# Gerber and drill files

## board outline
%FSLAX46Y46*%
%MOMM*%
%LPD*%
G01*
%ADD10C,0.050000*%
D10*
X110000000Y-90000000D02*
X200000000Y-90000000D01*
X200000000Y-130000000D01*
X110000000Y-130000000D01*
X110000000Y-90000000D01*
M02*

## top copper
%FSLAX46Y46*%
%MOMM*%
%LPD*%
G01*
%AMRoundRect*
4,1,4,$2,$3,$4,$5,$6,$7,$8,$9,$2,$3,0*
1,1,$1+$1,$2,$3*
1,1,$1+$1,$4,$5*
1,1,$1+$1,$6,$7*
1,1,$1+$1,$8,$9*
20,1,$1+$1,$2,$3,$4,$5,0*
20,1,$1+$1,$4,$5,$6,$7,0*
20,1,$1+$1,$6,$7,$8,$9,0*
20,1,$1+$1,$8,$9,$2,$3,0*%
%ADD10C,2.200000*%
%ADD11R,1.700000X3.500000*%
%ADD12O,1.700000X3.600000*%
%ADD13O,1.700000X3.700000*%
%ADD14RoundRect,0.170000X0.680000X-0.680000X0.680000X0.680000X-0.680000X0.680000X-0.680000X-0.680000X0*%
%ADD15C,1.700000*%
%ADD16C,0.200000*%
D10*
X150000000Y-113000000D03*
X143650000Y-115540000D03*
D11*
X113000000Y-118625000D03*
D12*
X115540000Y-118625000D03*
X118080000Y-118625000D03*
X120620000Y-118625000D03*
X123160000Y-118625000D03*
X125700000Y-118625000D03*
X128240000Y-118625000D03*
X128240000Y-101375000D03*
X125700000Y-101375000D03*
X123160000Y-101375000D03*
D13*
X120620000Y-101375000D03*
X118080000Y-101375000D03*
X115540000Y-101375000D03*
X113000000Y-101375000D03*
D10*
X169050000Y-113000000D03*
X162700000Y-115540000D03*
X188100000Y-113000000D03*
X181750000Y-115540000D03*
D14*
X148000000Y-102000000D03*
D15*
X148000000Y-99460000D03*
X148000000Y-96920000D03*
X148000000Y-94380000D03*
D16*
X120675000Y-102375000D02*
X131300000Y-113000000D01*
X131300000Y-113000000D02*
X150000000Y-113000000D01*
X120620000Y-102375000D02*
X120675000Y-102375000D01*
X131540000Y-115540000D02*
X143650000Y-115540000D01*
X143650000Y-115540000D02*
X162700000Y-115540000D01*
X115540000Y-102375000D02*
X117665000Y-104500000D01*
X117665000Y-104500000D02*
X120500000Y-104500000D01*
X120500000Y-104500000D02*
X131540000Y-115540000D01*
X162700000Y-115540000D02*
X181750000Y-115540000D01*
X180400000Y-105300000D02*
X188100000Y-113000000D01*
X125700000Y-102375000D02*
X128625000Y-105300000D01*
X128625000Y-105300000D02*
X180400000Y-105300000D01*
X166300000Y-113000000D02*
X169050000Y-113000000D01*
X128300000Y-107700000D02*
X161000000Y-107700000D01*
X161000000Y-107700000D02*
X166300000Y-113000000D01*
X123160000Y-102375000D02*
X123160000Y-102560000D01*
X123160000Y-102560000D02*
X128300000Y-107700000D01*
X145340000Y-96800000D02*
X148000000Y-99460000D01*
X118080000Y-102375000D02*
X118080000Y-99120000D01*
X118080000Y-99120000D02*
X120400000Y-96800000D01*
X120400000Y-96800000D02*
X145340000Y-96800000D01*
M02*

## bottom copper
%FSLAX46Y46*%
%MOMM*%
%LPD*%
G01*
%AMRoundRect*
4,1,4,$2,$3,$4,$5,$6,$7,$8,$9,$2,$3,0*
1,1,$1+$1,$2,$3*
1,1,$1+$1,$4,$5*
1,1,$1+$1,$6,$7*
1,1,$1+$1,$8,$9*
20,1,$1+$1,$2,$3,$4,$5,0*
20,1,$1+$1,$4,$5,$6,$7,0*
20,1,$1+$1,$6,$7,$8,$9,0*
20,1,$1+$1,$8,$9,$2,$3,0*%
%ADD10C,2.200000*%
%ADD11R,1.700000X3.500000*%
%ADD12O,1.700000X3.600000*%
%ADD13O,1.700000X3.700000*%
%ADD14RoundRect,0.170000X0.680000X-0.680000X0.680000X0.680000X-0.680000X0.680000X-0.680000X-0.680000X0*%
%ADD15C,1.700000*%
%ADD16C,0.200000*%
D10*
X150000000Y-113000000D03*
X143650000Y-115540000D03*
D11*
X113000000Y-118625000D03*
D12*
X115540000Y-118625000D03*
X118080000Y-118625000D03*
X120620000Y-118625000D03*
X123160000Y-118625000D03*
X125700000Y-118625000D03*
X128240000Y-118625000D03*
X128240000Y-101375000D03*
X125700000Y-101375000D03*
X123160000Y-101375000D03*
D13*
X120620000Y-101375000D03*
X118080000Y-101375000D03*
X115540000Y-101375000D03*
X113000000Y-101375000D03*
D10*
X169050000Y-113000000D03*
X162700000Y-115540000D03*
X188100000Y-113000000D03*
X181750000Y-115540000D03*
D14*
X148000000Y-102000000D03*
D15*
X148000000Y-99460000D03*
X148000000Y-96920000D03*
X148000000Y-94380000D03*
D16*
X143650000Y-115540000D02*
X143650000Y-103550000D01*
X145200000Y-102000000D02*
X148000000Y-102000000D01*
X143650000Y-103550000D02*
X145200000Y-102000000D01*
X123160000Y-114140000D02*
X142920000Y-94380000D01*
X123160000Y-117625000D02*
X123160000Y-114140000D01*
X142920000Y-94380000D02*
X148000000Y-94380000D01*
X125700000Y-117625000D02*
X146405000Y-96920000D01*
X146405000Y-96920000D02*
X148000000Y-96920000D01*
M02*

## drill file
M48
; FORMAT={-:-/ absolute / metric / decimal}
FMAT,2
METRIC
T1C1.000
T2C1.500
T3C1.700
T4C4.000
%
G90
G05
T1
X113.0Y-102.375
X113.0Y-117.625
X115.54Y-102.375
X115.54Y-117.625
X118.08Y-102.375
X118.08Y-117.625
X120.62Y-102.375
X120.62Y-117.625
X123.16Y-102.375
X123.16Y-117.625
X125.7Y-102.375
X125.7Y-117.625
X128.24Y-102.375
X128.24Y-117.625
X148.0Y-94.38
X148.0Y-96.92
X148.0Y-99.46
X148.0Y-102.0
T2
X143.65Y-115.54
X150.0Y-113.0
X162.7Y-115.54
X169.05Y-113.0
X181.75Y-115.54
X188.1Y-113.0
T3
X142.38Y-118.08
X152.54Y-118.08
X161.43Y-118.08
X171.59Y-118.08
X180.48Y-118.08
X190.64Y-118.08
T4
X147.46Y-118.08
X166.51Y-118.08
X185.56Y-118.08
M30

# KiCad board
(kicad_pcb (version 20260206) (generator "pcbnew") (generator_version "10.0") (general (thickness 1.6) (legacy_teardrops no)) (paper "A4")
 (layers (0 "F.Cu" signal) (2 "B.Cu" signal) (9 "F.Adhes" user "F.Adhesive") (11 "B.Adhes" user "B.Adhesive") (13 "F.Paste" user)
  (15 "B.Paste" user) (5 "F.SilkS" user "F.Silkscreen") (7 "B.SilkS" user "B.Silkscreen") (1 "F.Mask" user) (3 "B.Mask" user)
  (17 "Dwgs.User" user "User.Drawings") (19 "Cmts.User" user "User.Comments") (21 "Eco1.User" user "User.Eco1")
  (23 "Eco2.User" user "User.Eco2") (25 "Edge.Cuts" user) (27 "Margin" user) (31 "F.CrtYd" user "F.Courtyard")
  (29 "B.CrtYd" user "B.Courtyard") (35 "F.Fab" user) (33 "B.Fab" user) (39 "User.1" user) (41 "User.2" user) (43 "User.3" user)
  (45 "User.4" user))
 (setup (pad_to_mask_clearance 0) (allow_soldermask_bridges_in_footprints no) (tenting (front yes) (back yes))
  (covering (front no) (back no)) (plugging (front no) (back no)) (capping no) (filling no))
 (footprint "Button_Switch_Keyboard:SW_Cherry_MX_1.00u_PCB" (layer "F.Cu") (at 150 113)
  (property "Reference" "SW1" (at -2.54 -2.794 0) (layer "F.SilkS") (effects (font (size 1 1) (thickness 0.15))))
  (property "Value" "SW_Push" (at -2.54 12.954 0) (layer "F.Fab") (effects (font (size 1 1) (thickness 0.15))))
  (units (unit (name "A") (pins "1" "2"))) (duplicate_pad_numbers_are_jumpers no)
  (pad "" np_thru_hole circle (at -7.62 5.08) (size 1.7 1.7) (drill 1.7) (layers "*.Cu" "*.Mask"))
  (pad "" np_thru_hole circle (at -2.54 5.08) (size 4 4) (drill 4) (layers "*.Cu" "*.Mask"))
  (pad "" np_thru_hole circle (at 2.54 5.08) (size 1.7 1.7) (drill 1.7) (layers "*.Cu" "*.Mask"))
  (pad "1" thru_hole circle (at 0 0) (size 2.2 2.2) (drill 1.5) (layers "*.Cu" "*.Mask") (remove_unused_layers no)
   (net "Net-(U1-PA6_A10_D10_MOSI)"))
  (pad "2" thru_hole circle (at -6.35 2.54) (size 2.2 2.2) (drill 1.5) (layers "*.Cu" "*.Mask") (remove_unused_layers no) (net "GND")))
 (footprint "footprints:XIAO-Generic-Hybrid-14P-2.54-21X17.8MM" (layer "F.Cu") (at 120.62 110 90)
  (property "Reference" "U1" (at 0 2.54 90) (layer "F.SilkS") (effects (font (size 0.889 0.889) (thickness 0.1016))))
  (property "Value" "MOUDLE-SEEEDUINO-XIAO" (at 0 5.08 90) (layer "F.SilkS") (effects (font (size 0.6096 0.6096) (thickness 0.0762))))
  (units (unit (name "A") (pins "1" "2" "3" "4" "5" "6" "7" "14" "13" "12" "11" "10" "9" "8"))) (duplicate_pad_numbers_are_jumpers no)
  (pad "1" thru_hole rect (at -7.625 -7.62 90) (size 3.5 1.7) (drill 1 (offset -1 0)) (layers "*.Cu" "*.Mask") (remove_unused_layers no)
   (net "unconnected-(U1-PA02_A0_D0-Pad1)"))
  (pad "2" thru_hole oval (at -7.625 -5.08 90) (size 3.6 1.7) (drill 1 (offset -1 0)) (layers "*.Cu" "*.Mask") (remove_unused_layers no)
   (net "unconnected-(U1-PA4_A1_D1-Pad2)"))
  (pad "3" thru_hole oval (at -7.625 -2.54 90) (size 3.6 1.7) (drill 1 (offset -1 0)) (layers "*.Cu" "*.Mask") (remove_unused_layers no)
   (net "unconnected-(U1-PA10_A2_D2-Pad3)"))
  (pad "4" thru_hole oval (at -7.625 0 90) (size 3.6 1.7) (drill 1 (offset -1 0)) (layers "*.Cu" "*.Mask") (remove_unused_layers no)
   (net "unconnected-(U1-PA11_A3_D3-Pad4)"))
  (pad "5" thru_hole oval (at -7.625 2.54 90) (size 3.6 1.7) (drill 1 (offset -1 0)) (layers "*.Cu" "*.Mask") (remove_unused_layers no)
   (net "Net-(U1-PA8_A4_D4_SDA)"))
  (pad "6" thru_hole oval (at -7.625 5.08 270) (size 3.6 1.7) (drill 1 (offset 1 0)) (layers "*.Cu" "*.Mask") (remove_unused_layers no)
   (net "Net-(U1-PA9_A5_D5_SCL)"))
  (pad "7" thru_hole oval (at -7.625 7.62 90) (size 3.6 1.7) (drill 1 (offset -1 0)) (layers "*.Cu" "*.Mask") (remove_unused_layers no)
   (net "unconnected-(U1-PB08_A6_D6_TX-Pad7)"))
  (pad "8" thru_hole oval (at 7.625 7.62 90) (size 3.6 1.7) (drill 1 (offset 1 0)) (layers "*.Cu" "*.Mask") (remove_unused_layers no)
   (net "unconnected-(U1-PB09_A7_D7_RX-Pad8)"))
  (pad "9" thru_hole oval (at 7.625 5.08 90) (size 3.6 1.7) (drill 1 (offset 1 0)) (layers "*.Cu" "*.Mask") (remove_unused_layers no)
   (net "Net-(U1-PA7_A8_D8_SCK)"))
  (pad "10" thru_hole oval (at 7.625 2.54 90) (size 3.6 1.7) (drill 1 (offset 1 0)) (layers "*.Cu" "*.Mask") (remove_unused_layers no)
   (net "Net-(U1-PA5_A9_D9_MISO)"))
  (pad "11" thru_hole oval (at 7.625 0 90) (size 3.7 1.7) (drill 1 (offset 1 0)) (layers "*.Cu" "*.Mask") (remove_unused_layers no)
   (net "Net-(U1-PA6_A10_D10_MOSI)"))
  (pad "12" thru_hole oval (at 7.625 -2.54 90) (size 3.7 1.7) (drill 1 (offset 1 0)) (layers "*.Cu" "*.Mask") (remove_unused_layers no)
   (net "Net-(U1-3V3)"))
  (pad "13" thru_hole oval (at 7.625 -5.08 90) (size 3.7 1.7) (drill 1 (offset 1 0)) (layers "*.Cu" "*.Mask") (remove_unused_layers no)
   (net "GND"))
  (pad "14" thru_hole oval (at 7.625 -7.62 90) (size 3.7 1.7) (drill 1 (offset 1 0)) (layers "*.Cu" "*.Mask") (remove_unused_layers no)
   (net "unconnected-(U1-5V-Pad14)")))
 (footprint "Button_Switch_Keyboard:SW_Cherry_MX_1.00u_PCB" (layer "F.Cu") (at 169.05 113)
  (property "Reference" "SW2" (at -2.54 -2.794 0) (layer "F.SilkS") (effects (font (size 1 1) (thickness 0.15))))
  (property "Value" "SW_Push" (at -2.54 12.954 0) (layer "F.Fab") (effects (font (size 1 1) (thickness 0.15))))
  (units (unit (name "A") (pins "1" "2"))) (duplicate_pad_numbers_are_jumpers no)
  (pad "" np_thru_hole circle (at -7.62 5.08) (size 1.7 1.7) (drill 1.7) (layers "*.Cu" "*.Mask"))
  (pad "" np_thru_hole circle (at -2.54 5.08) (size 4 4) (drill 4) (layers "*.Cu" "*.Mask"))
  (pad "" np_thru_hole circle (at 2.54 5.08) (size 1.7 1.7) (drill 1.7) (layers "*.Cu" "*.Mask"))
  (pad "1" thru_hole circle (at 0 0) (size 2.2 2.2) (drill 1.5) (layers "*.Cu" "*.Mask") (remove_unused_layers no)
   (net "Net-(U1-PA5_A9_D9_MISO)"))
  (pad "2" thru_hole circle (at -6.35 2.54) (size 2.2 2.2) (drill 1.5) (layers "*.Cu" "*.Mask") (remove_unused_layers no) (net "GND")))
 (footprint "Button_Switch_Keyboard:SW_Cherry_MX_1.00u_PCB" (layer "F.Cu") (at 188.1 113)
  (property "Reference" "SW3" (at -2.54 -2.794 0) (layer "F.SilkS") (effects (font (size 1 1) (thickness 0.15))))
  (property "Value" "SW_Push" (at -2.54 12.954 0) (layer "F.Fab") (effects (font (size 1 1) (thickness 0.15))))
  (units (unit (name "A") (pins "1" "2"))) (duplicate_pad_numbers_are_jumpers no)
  (pad "" np_thru_hole circle (at -7.62 5.08) (size 1.7 1.7) (drill 1.7) (layers "*.Cu" "*.Mask"))
  (pad "" np_thru_hole circle (at -2.54 5.08) (size 4 4) (drill 4) (layers "*.Cu" "*.Mask"))
  (pad "" np_thru_hole circle (at 2.54 5.08) (size 1.7 1.7) (drill 1.7) (layers "*.Cu" "*.Mask"))
  (pad "1" thru_hole circle (at 0 0) (size 2.2 2.2) (drill 1.5) (layers "*.Cu" "*.Mask") (remove_unused_layers no)
   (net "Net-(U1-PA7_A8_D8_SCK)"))
  (pad "2" thru_hole circle (at -6.35 2.54) (size 2.2 2.2) (drill 1.5) (layers "*.Cu" "*.Mask") (remove_unused_layers no) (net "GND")))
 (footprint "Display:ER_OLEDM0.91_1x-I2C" (layer "F.Cu") (at 148 102 90)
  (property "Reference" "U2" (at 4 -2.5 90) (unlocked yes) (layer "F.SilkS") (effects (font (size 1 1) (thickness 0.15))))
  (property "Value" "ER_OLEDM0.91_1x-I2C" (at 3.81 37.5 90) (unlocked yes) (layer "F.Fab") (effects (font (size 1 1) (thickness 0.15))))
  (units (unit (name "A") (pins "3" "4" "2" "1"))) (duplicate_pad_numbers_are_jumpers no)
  (pad "1" thru_hole roundrect (at 0 0 90) (size 1.7 1.7) (drill 1) (layers "*.Cu" "*.Mask") (remove_unused_layers no)
   (roundrect_rratio 0.1) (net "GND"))
  (pad "2" thru_hole circle (at 2.54 0 90) (size 1.7 1.7) (drill 1) (layers "*.Cu" "*.Mask") (remove_unused_layers no) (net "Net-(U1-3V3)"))
  (pad "3" thru_hole circle (at 5.08 0 90) (size 1.7 1.7) (drill 1) (layers "*.Cu" "*.Mask") (remove_unused_layers no)
   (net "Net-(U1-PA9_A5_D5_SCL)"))
  (pad "4" thru_hole circle (at 7.62 0 90) (size 1.7 1.7) (drill 1) (layers "*.Cu" "*.Mask") (remove_unused_layers no)
   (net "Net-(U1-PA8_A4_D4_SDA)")))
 (gr_rect (start 110 90) (end 200 130) (stroke (width 0.05) (type default)) (fill no) (layer "Edge.Cuts"))
 (segment (start 120.675 102.375) (end 131.3 113) (width 0.2) (layer "F.Cu") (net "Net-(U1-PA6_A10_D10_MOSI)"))
 (segment (start 131.3 113) (end 150 113) (width 0.2) (layer "F.Cu") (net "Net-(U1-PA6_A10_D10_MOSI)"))
 (segment (start 120.62 102.375) (end 120.675 102.375) (width 0.2) (layer "F.Cu") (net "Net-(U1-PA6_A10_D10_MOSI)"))
 (segment (start 131.54 115.54) (end 143.65 115.54) (width 0.2) (layer "F.Cu") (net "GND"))
 (segment (start 143.65 115.54) (end 162.7 115.54) (width 0.2) (layer "F.Cu") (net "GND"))
 (segment (start 115.54 102.375) (end 117.665 104.5) (width 0.2) (layer "F.Cu") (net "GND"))
 (segment (start 117.665 104.5) (end 120.5 104.5) (width 0.2) (layer "F.Cu") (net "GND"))
 (segment (start 120.5 104.5) (end 131.54 115.54) (width 0.2) (layer "F.Cu") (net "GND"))
 (segment (start 162.7 115.54) (end 181.75 115.54) (width 0.2) (layer "F.Cu") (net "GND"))
 (segment (start 143.65 115.54) (end 143.65 103.55) (width 0.2) (layer "B.Cu") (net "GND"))
 (segment (start 145.2 102) (end 148 102) (width 0.2) (layer "B.Cu") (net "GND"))
 (segment (start 143.65 103.55) (end 145.2 102) (width 0.2) (layer "B.Cu") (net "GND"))
 (segment (start 123.16 114.14) (end 142.92 94.38) (width 0.2) (layer "B.Cu") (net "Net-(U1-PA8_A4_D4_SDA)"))
 (segment (start 123.16 117.625) (end 123.16 114.14) (width 0.2) (layer "B.Cu") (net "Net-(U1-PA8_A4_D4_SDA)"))
 (segment (start 142.92 94.38) (end 148 94.38) (width 0.2) (layer "B.Cu") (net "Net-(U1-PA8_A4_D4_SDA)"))
 (segment (start 125.7 117.625) (end 146.405 96.92) (width 0.2) (layer "B.Cu") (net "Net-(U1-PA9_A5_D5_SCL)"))
 (segment (start 146.405 96.92) (end 148 96.92) (width 0.2) (layer "B.Cu") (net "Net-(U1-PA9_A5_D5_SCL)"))
 (segment (start 180.4 105.3) (end 188.1 113) (width 0.2) (layer "F.Cu") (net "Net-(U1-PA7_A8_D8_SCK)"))
 (segment (start 125.7 102.375) (end 128.625 105.3) (width 0.2) (layer "F.Cu") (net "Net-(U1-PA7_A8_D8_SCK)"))
 (segment (start 128.625 105.3) (end 180.4 105.3) (width 0.2) (layer "F.Cu") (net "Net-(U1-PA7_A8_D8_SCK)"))
 (segment (start 166.3 113) (end 169.05 113) (width 0.2) (layer "F.Cu") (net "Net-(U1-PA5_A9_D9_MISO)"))
 (segment (start 128.3 107.7) (end 161 107.7) (width 0.2) (layer "F.Cu") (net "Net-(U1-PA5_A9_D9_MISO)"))
 (segment (start 161 107.7) (end 166.3 113) (width 0.2) (layer "F.Cu") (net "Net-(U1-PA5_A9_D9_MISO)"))
 (segment (start 123.16 102.375) (end 123.16 102.56) (width 0.2) (layer "F.Cu") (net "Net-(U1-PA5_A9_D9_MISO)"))
 (segment (start 123.16 102.56) (end 128.3 107.7) (width 0.2) (layer "F.Cu") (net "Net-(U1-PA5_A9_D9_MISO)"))
 (segment (start 145.34 96.8) (end 148 99.46) (width 0.2) (layer "F.Cu") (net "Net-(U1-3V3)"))
 (segment (start 118.08 102.375) (end 118.08 99.12) (width 0.2) (layer "F.Cu") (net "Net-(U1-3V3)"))
 (segment (start 118.08 99.12) (end 120.4 96.8) (width 0.2) (layer "F.Cu") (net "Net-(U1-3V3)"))
 (segment (start 120.4 96.8) (end 145.34 96.8) (width 0.2) (layer "F.Cu") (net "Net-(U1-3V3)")))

